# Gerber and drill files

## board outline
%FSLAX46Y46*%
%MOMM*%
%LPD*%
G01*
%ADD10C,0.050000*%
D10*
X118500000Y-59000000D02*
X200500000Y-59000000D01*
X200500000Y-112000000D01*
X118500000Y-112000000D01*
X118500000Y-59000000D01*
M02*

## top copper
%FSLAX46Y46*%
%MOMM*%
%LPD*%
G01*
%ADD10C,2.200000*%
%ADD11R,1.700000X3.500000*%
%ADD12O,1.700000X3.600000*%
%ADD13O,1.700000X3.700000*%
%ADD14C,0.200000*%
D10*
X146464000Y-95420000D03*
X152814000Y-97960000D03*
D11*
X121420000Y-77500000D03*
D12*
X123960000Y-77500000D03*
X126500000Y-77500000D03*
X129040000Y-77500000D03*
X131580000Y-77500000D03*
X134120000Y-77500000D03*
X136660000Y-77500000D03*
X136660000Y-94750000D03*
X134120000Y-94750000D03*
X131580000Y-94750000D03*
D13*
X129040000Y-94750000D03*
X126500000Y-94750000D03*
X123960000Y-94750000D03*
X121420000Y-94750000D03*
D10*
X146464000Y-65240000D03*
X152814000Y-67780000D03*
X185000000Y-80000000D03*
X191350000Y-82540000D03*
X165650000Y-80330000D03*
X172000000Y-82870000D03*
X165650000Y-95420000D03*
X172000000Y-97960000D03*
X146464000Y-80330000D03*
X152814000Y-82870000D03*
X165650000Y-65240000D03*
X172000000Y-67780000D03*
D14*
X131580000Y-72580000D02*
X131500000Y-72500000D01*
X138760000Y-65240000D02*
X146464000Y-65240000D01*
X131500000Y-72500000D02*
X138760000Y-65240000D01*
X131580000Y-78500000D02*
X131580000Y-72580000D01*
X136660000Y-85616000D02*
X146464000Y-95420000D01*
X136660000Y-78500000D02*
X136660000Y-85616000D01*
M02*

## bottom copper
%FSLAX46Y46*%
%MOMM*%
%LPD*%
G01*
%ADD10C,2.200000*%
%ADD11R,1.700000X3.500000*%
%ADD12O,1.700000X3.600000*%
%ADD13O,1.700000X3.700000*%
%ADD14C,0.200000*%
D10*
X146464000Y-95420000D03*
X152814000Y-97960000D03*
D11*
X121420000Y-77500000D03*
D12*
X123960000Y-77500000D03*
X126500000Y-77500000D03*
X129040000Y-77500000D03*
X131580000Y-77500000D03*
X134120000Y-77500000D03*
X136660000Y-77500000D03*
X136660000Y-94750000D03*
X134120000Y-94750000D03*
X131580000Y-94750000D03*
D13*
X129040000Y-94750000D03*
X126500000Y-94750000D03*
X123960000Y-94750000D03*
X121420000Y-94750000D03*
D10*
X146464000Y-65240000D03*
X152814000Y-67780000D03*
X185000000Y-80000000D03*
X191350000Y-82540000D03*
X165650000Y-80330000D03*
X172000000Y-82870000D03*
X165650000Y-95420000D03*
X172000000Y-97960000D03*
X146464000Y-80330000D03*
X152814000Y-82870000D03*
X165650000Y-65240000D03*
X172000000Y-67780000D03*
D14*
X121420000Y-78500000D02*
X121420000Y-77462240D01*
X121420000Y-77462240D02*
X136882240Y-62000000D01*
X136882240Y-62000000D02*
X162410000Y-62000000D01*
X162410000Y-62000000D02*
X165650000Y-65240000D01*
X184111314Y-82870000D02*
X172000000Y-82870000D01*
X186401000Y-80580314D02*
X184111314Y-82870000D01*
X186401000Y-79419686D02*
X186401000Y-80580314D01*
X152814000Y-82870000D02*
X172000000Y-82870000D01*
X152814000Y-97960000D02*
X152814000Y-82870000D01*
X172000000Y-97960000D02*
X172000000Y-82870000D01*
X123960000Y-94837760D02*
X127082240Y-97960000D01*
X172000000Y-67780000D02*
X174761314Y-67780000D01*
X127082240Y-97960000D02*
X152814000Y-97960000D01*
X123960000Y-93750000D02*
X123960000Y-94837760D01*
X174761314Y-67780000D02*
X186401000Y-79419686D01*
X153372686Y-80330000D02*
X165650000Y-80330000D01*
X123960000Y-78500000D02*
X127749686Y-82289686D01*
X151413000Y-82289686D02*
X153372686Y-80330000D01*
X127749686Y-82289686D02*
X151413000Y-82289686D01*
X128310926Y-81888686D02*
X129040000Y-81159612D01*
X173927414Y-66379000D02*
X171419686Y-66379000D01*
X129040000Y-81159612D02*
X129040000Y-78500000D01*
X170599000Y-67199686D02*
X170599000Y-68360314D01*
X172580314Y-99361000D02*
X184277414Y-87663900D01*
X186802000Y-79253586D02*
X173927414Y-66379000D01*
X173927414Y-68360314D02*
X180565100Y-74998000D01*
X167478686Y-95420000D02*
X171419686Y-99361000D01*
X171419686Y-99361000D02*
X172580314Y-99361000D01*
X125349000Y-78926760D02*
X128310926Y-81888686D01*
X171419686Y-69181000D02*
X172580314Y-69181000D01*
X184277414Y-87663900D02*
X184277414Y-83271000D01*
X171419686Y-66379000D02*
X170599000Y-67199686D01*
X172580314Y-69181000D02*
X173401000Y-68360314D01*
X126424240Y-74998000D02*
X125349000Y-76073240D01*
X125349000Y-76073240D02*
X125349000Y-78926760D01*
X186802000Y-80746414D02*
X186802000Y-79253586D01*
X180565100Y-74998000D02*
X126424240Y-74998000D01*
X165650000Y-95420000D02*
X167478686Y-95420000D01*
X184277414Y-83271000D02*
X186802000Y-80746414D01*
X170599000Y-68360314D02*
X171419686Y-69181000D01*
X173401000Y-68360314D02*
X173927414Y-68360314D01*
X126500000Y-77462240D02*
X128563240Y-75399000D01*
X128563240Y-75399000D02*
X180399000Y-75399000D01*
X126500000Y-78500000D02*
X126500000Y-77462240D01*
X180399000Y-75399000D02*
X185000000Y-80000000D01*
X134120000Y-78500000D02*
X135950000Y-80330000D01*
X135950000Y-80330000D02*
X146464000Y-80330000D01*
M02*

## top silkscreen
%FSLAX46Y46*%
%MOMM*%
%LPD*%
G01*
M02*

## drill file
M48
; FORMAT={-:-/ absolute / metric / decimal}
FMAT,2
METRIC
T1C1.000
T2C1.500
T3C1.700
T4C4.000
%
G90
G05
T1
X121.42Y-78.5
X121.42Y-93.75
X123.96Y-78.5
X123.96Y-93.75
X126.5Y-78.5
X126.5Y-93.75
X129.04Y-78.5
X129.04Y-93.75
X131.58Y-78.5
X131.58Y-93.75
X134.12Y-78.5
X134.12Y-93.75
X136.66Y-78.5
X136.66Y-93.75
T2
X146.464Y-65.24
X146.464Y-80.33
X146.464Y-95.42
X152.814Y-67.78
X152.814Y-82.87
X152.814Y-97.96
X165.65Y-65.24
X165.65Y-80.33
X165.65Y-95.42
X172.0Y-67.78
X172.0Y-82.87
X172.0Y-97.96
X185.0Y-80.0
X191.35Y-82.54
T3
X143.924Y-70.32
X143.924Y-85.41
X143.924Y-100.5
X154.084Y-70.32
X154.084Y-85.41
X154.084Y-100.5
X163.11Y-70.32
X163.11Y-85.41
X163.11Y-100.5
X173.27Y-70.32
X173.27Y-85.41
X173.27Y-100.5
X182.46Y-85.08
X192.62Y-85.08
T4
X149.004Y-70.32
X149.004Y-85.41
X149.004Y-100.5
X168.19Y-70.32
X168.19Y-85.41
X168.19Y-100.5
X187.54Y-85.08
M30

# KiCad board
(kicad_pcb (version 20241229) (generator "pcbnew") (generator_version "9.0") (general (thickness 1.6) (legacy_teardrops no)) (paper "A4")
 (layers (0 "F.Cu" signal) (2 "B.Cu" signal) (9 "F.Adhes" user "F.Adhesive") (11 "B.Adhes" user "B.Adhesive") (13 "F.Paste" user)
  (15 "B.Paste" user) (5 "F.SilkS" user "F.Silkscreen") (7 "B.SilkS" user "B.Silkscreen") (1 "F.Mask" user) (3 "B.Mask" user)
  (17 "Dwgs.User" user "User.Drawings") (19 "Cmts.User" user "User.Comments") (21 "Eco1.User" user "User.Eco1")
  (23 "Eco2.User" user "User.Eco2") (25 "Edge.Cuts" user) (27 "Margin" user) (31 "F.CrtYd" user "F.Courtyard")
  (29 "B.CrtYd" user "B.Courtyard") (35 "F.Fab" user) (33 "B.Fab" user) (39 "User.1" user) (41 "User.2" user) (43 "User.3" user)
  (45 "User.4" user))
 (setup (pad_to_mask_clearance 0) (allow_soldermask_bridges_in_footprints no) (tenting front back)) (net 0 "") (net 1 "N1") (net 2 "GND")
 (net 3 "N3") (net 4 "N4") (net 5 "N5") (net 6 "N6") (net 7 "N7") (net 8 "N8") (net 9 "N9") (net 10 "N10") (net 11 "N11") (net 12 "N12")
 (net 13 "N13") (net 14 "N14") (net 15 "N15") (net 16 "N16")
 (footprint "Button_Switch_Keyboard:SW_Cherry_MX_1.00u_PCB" (layer "B.Cu") (at 146.464 95.42 180)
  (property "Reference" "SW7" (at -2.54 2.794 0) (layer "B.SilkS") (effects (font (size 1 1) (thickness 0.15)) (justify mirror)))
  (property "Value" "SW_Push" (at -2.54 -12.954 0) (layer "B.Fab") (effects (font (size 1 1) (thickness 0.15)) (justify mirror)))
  (pad "" np_thru_hole circle (at -7.62 -5.08 180) (size 1.7 1.7) (drill 1.7) (layers "*.Cu" "*.Mask"))
  (pad "" np_thru_hole circle (at -2.54 -5.08 180) (size 4 4) (drill 4) (layers "*.Cu" "*.Mask"))
  (pad "" np_thru_hole circle (at 2.54 -5.08 180) (size 1.7 1.7) (drill 1.7) (layers "*.Cu" "*.Mask"))
  (pad "1" thru_hole circle (at 0 0 180) (size 2.2 2.2) (drill 1.5) (layers "*.Cu" "*.Mask") (remove_unused_layers no) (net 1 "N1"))
  (pad "2" thru_hole circle (at -6.35 -2.54 180) (size 2.2 2.2) (drill 1.5) (layers "*.Cu" "*.Mask") (remove_unused_layers no) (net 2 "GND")))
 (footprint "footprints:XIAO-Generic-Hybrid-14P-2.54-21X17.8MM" (layer "B.Cu") (at 129.04 86.125 -90)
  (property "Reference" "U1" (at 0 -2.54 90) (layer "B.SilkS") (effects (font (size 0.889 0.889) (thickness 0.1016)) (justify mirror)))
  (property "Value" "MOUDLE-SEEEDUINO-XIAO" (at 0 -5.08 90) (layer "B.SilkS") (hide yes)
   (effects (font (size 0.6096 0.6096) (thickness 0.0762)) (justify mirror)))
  (pad "1" thru_hole rect (at -7.625 7.62 270) (size 3.5 1.7) (drill 1 (offset -1 0)) (layers "*.Cu" "*.Mask") (remove_unused_layers no)
   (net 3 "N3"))
  (pad "2" thru_hole oval (at -7.625 5.08 270) (size 3.6 1.7) (drill 1 (offset -1 0)) (layers "*.Cu" "*.Mask") (remove_unused_layers no)
   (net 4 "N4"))
  (pad "3" thru_hole oval (at -7.625 2.54 270) (size 3.6 1.7) (drill 1 (offset -1 0)) (layers "*.Cu" "*.Mask") (remove_unused_layers no)
   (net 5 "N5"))
  (pad "4" thru_hole oval (at -7.625 0 270) (size 3.6 1.7) (drill 1 (offset -1 0)) (layers "*.Cu" "*.Mask") (remove_unused_layers no)
   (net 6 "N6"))
  (pad "5" thru_hole oval (at -7.625 -2.54 270) (size 3.6 1.7) (drill 1 (offset -1 0)) (layers "*.Cu" "*.Mask") (remove_unused_layers no)
   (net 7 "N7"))
  (pad "6" thru_hole oval (at -7.625 -5.08 90) (size 3.6 1.7) (drill 1 (offset 1 0)) (layers "*.Cu" "*.Mask") (remove_unused_layers no)
   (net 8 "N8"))
  (pad "7" thru_hole oval (at -7.625 -7.62 270) (size 3.6 1.7) (drill 1 (offset -1 0)) (layers "*.Cu" "*.Mask") (remove_unused_layers no)
   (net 1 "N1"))
  (pad "8" thru_hole oval (at 7.625 -7.62 270) (size 3.6 1.7) (drill 1 (offset 1 0)) (layers "*.Cu" "*.Mask") (remove_unused_layers no)
   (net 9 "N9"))
  (pad "9" thru_hole oval (at 7.625 -5.08 270) (size 3.6 1.7) (drill 1 (offset 1 0)) (layers "*.Cu" "*.Mask") (remove_unused_layers no)
   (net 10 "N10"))
  (pad "10" thru_hole oval (at 7.625 -2.54 270) (size 3.6 1.7) (drill 1 (offset 1 0)) (layers "*.Cu" "*.Mask") (remove_unused_layers no)
   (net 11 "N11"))
  (pad "11" thru_hole oval (at 7.625 0 270) (size 3.7 1.7) (drill 1 (offset 1 0)) (layers "*.Cu" "*.Mask") (remove_unused_layers no)
   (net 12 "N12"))
  (pad "12" thru_hole oval (at 7.625 2.54 270) (size 3.7 1.7) (drill 1 (offset 1 0)) (layers "*.Cu" "*.Mask") (remove_unused_layers no)
   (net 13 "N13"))
  (pad "13" thru_hole oval (at 7.625 5.08 270) (size 3.7 1.7) (drill 1 (offset 1 0)) (layers "*.Cu" "*.Mask") (remove_unused_layers no)
   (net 2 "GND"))
  (pad "14" thru_hole oval (at 7.625 7.62 270) (size 3.7 1.7) (drill 1 (offset 1 0)) (layers "*.Cu" "*.Mask") (remove_unused_layers no)
   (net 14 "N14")))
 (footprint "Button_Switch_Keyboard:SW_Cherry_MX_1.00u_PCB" (layer "B.Cu") (at 146.464 65.24 180)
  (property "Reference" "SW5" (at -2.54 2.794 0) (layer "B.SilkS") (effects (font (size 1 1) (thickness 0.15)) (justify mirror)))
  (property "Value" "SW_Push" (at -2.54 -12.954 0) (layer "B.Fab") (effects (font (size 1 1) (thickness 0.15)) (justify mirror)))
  (pad "" np_thru_hole circle (at -7.62 -5.08 180) (size 1.7 1.7) (drill 1.7) (layers "*.Cu" "*.Mask"))
  (pad "" np_thru_hole circle (at -2.54 -5.08 180) (size 4 4) (drill 4) (layers "*.Cu" "*.Mask"))
  (pad "" np_thru_hole circle (at 2.54 -5.08 180) (size 1.7 1.7) (drill 1.7) (layers "*.Cu" "*.Mask"))
  (pad "1" thru_hole circle (at 0 0 180) (size 2.2 2.2) (drill 1.5) (layers "*.Cu" "*.Mask") (remove_unused_layers no) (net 7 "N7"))
  (pad "2" thru_hole circle (at -6.35 -2.54 180) (size 2.2 2.2) (drill 1.5) (layers "*.Cu" "*.Mask") (remove_unused_layers no)
   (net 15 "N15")))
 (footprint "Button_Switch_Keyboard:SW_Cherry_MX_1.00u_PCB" (layer "B.Cu") (at 185 80 180)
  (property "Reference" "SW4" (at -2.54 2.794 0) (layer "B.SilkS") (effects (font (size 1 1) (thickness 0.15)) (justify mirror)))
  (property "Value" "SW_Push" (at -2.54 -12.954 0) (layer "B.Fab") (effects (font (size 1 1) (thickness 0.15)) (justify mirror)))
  (pad "" np_thru_hole circle (at -7.62 -5.08 180) (size 1.7 1.7) (drill 1.7) (layers "*.Cu" "*.Mask"))
  (pad "" np_thru_hole circle (at -2.54 -5.08 180) (size 4 4) (drill 4) (layers "*.Cu" "*.Mask"))
  (pad "" np_thru_hole circle (at 2.54 -5.08 180) (size 1.7 1.7) (drill 1.7) (layers "*.Cu" "*.Mask"))
  (pad "1" thru_hole circle (at 0 0 180) (size 2.2 2.2) (drill 1.5) (layers "*.Cu" "*.Mask") (remove_unused_layers no) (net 5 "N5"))
  (pad "2" thru_hole circle (at -6.35 -2.54 180) (size 2.2 2.2) (drill 1.5) (layers "*.Cu" "*.Mask") (remove_unused_layers no)
   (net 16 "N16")))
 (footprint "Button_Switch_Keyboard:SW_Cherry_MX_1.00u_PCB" (layer "B.Cu") (at 165.65 80.33 180)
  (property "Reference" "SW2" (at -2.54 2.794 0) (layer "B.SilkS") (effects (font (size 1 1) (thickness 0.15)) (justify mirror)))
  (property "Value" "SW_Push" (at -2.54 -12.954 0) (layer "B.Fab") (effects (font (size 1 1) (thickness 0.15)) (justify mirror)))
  (pad "" np_thru_hole circle (at -7.62 -5.08 180) (size 1.7 1.7) (drill 1.7) (layers "*.Cu" "*.Mask"))
  (pad "" np_thru_hole circle (at -2.54 -5.08 180) (size 4 4) (drill 4) (layers "*.Cu" "*.Mask"))
  (pad "" np_thru_hole circle (at 2.54 -5.08 180) (size 1.7 1.7) (drill 1.7) (layers "*.Cu" "*.Mask"))
  (pad "1" thru_hole circle (at 0 0 180) (size 2.2 2.2) (drill 1.5) (layers "*.Cu" "*.Mask") (remove_unused_layers no) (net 4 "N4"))
  (pad "2" thru_hole circle (at -6.35 -2.54 180) (size 2.2 2.2) (drill 1.5) (layers "*.Cu" "*.Mask") (remove_unused_layers no) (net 2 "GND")))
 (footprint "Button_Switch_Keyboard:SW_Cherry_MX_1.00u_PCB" (layer "B.Cu") (at 165.65 95.42 180)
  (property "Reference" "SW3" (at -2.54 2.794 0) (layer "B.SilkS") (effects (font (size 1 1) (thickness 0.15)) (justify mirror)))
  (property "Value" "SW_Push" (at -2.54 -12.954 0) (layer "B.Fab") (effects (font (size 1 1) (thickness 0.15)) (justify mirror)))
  (pad "" np_thru_hole circle (at -7.62 -5.08 180) (size 1.7 1.7) (drill 1.7) (layers "*.Cu" "*.Mask"))
  (pad "" np_thru_hole circle (at -2.54 -5.08 180) (size 4 4) (drill 4) (layers "*.Cu" "*.Mask"))
  (pad "" np_thru_hole circle (at 2.54 -5.08 180) (size 1.7 1.7) (drill 1.7) (layers "*.Cu" "*.Mask"))
  (pad "1" thru_hole circle (at 0 0 180) (size 2.2 2.2) (drill 1.5) (layers "*.Cu" "*.Mask") (remove_unused_layers no) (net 6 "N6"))
  (pad "2" thru_hole circle (at -6.35 -2.54 180) (size 2.2 2.2) (drill 1.5) (layers "*.Cu" "*.Mask") (remove_unused_layers no) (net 2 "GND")))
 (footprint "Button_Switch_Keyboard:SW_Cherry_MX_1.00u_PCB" (layer "B.Cu") (at 146.464 80.33 180)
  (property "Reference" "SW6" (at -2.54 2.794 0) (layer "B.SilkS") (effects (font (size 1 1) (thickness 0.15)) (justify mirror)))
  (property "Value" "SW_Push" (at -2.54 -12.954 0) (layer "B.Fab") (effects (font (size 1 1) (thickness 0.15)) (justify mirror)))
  (pad "" np_thru_hole circle (at -7.62 -5.08 180) (size 1.7 1.7) (drill 1.7) (layers "*.Cu" "*.Mask"))
  (pad "" np_thru_hole circle (at -2.54 -5.08 180) (size 4 4) (drill 4) (layers "*.Cu" "*.Mask"))
  (pad "" np_thru_hole circle (at 2.54 -5.08 180) (size 1.7 1.7) (drill 1.7) (layers "*.Cu" "*.Mask"))
  (pad "1" thru_hole circle (at 0 0 180) (size 2.2 2.2) (drill 1.5) (layers "*.Cu" "*.Mask") (remove_unused_layers no) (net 8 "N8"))
  (pad "2" thru_hole circle (at -6.35 -2.54 180) (size 2.2 2.2) (drill 1.5) (layers "*.Cu" "*.Mask") (remove_unused_layers no) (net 2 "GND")))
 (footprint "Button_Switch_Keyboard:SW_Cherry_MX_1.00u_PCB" (layer "B.Cu") (at 165.65 65.24 180)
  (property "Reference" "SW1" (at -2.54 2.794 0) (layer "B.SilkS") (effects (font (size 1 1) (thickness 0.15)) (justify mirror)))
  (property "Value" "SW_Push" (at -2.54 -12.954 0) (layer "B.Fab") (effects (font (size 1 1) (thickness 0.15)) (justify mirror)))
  (pad "" np_thru_hole circle (at -7.62 -5.08 180) (size 1.7 1.7) (drill 1.7) (layers "*.Cu" "*.Mask"))
  (pad "" np_thru_hole circle (at -2.54 -5.08 180) (size 4 4) (drill 4) (layers "*.Cu" "*.Mask"))
  (pad "" np_thru_hole circle (at 2.54 -5.08 180) (size 1.7 1.7) (drill 1.7) (layers "*.Cu" "*.Mask"))
  (pad "1" thru_hole circle (at 0 0 180) (size 2.2 2.2) (drill 1.5) (layers "*.Cu" "*.Mask") (remove_unused_layers no) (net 3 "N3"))
  (pad "2" thru_hole circle (at -6.35 -2.54 180) (size 2.2 2.2) (drill 1.5) (layers "*.Cu" "*.Mask") (remove_unused_layers no) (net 2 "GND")))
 (gr_rect (start 118.5 59) (end 200.5 112) (stroke (width 0.05) (type default)) (fill no) (layer "Edge.Cuts"))
 (segment (start 121.42 78.5) (end 121.42 77.46224) (width 0.2) (layer "B.Cu") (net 3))
 (segment (start 121.42 77.46224) (end 136.88224 62) (width 0.2) (layer "B.Cu") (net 3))
 (segment (start 136.88224 62) (end 162.41 62) (width 0.2) (layer "B.Cu") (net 3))
 (segment (start 162.41 62) (end 165.65 65.24) (width 0.2) (layer "B.Cu") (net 3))
 (segment (start 184.111314 82.87) (end 172 82.87) (width 0.2) (layer "B.Cu") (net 2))
 (segment (start 186.401 80.580314) (end 184.111314 82.87) (width 0.2) (layer "B.Cu") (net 2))
 (segment (start 186.401 79.419686) (end 186.401 80.580314) (width 0.2) (layer "B.Cu") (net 2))
 (segment (start 152.814 82.87) (end 172 82.87) (width 0.2) (layer "B.Cu") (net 2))
 (segment (start 152.814 97.96) (end 152.814 82.87) (width 0.2) (layer "B.Cu") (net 2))
 (segment (start 172 97.96) (end 172 82.87) (width 0.2) (layer "B.Cu") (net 2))
 (segment (start 123.96 94.83776) (end 127.08224 97.96) (width 0.2) (layer "B.Cu") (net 2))
 (segment (start 172 67.78) (end 174.761314 67.78) (width 0.2) (layer "B.Cu") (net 2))
 (segment (start 127.08224 97.96) (end 152.814 97.96) (width 0.2) (layer "B.Cu") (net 2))
 (segment (start 123.96 93.75) (end 123.96 94.83776) (width 0.2) (layer "B.Cu") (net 2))
 (segment (start 174.761314 67.78) (end 186.401 79.419686) (width 0.2) (layer "B.Cu") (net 2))
 (segment (start 153.372686 80.33) (end 165.65 80.33) (width 0.2) (layer "B.Cu") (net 4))
 (segment (start 123.96 78.5) (end 127.749686 82.289686) (width 0.2) (layer "B.Cu") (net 4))
 (segment (start 151.413 82.289686) (end 153.372686 80.33) (width 0.2) (layer "B.Cu") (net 4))
 (segment (start 127.749686 82.289686) (end 151.413 82.289686) (width 0.2) (layer "B.Cu") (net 4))
 (segment (start 128.310926 81.888686) (end 129.04 81.159612) (width 0.2) (layer "B.Cu") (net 6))
 (segment (start 173.927414 66.379) (end 171.419686 66.379) (width 0.2) (layer "B.Cu") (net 6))
 (segment (start 129.04 81.159612) (end 129.04 78.5) (width 0.2) (layer "B.Cu") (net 6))
 (segment (start 170.599 67.199686) (end 170.599 68.360314) (width 0.2) (layer "B.Cu") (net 6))
 (segment (start 172.580314 99.361) (end 184.277414 87.6639) (width 0.2) (layer "B.Cu") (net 6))
 (segment (start 186.802 79.253586) (end 173.927414 66.379) (width 0.2) (layer "B.Cu") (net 6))
 (segment (start 173.927414 68.360314) (end 180.5651 74.998) (width 0.2) (layer "B.Cu") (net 6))
 (segment (start 167.478686 95.42) (end 171.419686 99.361) (width 0.2) (layer "B.Cu") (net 6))
 (segment (start 171.419686 99.361) (end 172.580314 99.361) (width 0.2) (layer "B.Cu") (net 6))
 (segment (start 125.349 78.92676) (end 128.310926 81.888686) (width 0.2) (layer "B.Cu") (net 6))
 (segment (start 171.419686 69.181) (end 172.580314 69.181) (width 0.2) (layer "B.Cu") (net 6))
 (segment (start 184.277414 87.6639) (end 184.277414 83.271) (width 0.2) (layer "B.Cu") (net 6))
 (segment (start 171.419686 66.379) (end 170.599 67.199686) (width 0.2) (layer "B.Cu") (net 6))
 (segment (start 172.580314 69.181) (end 173.401 68.360314) (width 0.2) (layer "B.Cu") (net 6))
 (segment (start 126.42424 74.998) (end 125.349 76.07324) (width 0.2) (layer "B.Cu") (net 6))
 (segment (start 125.349 76.07324) (end 125.349 78.92676) (width 0.2) (layer "B.Cu") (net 6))
 (segment (start 186.802 80.746414) (end 186.802 79.253586) (width 0.2) (layer "B.Cu") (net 6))
 (segment (start 180.5651 74.998) (end 126.42424 74.998) (width 0.2) (layer "B.Cu") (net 6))
 (segment (start 165.65 95.42) (end 167.478686 95.42) (width 0.2) (layer "B.Cu") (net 6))
 (segment (start 184.277414 83.271) (end 186.802 80.746414) (width 0.2) (layer "B.Cu") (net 6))
 (segment (start 170.599 68.360314) (end 171.419686 69.181) (width 0.2) (layer "B.Cu") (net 6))
 (segment (start 173.401 68.360314) (end 173.927414 68.360314) (width 0.2) (layer "B.Cu") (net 6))
 (segment (start 126.5 77.46224) (end 128.56324 75.399) (width 0.2) (layer "B.Cu") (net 5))
 (segment (start 128.56324 75.399) (end 180.399 75.399) (width 0.2) (layer "B.Cu") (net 5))
 (segment (start 126.5 78.5) (end 126.5 77.46224) (width 0.2) (layer "B.Cu") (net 5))
 (segment (start 180.399 75.399) (end 185 80) (width 0.2) (layer "B.Cu") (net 5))
 (segment (start 131.58 72.58) (end 131.5 72.5) (width 0.2) (layer "F.Cu") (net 7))
 (segment (start 138.76 65.24) (end 146.464 65.24) (width 0.2) (layer "F.Cu") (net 7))
 (segment (start 131.5 72.5) (end 138.76 65.24) (width 0.2) (layer "F.Cu") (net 7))
 (segment (start 131.58 78.5) (end 131.58 72.58) (width 0.2) (layer "F.Cu") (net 7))
 (segment (start 134.12 78.5) (end 135.95 80.33) (width 0.2) (layer "B.Cu") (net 8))
 (segment (start 135.95 80.33) (end 146.464 80.33) (width 0.2) (layer "B.Cu") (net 8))
 (segment (start 136.66 85.616) (end 146.464 95.42) (width 0.2) (layer "F.Cu") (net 1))
 (segment (start 136.66 78.5) (end 136.66 85.616) (width 0.2) (layer "F.Cu") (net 1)))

